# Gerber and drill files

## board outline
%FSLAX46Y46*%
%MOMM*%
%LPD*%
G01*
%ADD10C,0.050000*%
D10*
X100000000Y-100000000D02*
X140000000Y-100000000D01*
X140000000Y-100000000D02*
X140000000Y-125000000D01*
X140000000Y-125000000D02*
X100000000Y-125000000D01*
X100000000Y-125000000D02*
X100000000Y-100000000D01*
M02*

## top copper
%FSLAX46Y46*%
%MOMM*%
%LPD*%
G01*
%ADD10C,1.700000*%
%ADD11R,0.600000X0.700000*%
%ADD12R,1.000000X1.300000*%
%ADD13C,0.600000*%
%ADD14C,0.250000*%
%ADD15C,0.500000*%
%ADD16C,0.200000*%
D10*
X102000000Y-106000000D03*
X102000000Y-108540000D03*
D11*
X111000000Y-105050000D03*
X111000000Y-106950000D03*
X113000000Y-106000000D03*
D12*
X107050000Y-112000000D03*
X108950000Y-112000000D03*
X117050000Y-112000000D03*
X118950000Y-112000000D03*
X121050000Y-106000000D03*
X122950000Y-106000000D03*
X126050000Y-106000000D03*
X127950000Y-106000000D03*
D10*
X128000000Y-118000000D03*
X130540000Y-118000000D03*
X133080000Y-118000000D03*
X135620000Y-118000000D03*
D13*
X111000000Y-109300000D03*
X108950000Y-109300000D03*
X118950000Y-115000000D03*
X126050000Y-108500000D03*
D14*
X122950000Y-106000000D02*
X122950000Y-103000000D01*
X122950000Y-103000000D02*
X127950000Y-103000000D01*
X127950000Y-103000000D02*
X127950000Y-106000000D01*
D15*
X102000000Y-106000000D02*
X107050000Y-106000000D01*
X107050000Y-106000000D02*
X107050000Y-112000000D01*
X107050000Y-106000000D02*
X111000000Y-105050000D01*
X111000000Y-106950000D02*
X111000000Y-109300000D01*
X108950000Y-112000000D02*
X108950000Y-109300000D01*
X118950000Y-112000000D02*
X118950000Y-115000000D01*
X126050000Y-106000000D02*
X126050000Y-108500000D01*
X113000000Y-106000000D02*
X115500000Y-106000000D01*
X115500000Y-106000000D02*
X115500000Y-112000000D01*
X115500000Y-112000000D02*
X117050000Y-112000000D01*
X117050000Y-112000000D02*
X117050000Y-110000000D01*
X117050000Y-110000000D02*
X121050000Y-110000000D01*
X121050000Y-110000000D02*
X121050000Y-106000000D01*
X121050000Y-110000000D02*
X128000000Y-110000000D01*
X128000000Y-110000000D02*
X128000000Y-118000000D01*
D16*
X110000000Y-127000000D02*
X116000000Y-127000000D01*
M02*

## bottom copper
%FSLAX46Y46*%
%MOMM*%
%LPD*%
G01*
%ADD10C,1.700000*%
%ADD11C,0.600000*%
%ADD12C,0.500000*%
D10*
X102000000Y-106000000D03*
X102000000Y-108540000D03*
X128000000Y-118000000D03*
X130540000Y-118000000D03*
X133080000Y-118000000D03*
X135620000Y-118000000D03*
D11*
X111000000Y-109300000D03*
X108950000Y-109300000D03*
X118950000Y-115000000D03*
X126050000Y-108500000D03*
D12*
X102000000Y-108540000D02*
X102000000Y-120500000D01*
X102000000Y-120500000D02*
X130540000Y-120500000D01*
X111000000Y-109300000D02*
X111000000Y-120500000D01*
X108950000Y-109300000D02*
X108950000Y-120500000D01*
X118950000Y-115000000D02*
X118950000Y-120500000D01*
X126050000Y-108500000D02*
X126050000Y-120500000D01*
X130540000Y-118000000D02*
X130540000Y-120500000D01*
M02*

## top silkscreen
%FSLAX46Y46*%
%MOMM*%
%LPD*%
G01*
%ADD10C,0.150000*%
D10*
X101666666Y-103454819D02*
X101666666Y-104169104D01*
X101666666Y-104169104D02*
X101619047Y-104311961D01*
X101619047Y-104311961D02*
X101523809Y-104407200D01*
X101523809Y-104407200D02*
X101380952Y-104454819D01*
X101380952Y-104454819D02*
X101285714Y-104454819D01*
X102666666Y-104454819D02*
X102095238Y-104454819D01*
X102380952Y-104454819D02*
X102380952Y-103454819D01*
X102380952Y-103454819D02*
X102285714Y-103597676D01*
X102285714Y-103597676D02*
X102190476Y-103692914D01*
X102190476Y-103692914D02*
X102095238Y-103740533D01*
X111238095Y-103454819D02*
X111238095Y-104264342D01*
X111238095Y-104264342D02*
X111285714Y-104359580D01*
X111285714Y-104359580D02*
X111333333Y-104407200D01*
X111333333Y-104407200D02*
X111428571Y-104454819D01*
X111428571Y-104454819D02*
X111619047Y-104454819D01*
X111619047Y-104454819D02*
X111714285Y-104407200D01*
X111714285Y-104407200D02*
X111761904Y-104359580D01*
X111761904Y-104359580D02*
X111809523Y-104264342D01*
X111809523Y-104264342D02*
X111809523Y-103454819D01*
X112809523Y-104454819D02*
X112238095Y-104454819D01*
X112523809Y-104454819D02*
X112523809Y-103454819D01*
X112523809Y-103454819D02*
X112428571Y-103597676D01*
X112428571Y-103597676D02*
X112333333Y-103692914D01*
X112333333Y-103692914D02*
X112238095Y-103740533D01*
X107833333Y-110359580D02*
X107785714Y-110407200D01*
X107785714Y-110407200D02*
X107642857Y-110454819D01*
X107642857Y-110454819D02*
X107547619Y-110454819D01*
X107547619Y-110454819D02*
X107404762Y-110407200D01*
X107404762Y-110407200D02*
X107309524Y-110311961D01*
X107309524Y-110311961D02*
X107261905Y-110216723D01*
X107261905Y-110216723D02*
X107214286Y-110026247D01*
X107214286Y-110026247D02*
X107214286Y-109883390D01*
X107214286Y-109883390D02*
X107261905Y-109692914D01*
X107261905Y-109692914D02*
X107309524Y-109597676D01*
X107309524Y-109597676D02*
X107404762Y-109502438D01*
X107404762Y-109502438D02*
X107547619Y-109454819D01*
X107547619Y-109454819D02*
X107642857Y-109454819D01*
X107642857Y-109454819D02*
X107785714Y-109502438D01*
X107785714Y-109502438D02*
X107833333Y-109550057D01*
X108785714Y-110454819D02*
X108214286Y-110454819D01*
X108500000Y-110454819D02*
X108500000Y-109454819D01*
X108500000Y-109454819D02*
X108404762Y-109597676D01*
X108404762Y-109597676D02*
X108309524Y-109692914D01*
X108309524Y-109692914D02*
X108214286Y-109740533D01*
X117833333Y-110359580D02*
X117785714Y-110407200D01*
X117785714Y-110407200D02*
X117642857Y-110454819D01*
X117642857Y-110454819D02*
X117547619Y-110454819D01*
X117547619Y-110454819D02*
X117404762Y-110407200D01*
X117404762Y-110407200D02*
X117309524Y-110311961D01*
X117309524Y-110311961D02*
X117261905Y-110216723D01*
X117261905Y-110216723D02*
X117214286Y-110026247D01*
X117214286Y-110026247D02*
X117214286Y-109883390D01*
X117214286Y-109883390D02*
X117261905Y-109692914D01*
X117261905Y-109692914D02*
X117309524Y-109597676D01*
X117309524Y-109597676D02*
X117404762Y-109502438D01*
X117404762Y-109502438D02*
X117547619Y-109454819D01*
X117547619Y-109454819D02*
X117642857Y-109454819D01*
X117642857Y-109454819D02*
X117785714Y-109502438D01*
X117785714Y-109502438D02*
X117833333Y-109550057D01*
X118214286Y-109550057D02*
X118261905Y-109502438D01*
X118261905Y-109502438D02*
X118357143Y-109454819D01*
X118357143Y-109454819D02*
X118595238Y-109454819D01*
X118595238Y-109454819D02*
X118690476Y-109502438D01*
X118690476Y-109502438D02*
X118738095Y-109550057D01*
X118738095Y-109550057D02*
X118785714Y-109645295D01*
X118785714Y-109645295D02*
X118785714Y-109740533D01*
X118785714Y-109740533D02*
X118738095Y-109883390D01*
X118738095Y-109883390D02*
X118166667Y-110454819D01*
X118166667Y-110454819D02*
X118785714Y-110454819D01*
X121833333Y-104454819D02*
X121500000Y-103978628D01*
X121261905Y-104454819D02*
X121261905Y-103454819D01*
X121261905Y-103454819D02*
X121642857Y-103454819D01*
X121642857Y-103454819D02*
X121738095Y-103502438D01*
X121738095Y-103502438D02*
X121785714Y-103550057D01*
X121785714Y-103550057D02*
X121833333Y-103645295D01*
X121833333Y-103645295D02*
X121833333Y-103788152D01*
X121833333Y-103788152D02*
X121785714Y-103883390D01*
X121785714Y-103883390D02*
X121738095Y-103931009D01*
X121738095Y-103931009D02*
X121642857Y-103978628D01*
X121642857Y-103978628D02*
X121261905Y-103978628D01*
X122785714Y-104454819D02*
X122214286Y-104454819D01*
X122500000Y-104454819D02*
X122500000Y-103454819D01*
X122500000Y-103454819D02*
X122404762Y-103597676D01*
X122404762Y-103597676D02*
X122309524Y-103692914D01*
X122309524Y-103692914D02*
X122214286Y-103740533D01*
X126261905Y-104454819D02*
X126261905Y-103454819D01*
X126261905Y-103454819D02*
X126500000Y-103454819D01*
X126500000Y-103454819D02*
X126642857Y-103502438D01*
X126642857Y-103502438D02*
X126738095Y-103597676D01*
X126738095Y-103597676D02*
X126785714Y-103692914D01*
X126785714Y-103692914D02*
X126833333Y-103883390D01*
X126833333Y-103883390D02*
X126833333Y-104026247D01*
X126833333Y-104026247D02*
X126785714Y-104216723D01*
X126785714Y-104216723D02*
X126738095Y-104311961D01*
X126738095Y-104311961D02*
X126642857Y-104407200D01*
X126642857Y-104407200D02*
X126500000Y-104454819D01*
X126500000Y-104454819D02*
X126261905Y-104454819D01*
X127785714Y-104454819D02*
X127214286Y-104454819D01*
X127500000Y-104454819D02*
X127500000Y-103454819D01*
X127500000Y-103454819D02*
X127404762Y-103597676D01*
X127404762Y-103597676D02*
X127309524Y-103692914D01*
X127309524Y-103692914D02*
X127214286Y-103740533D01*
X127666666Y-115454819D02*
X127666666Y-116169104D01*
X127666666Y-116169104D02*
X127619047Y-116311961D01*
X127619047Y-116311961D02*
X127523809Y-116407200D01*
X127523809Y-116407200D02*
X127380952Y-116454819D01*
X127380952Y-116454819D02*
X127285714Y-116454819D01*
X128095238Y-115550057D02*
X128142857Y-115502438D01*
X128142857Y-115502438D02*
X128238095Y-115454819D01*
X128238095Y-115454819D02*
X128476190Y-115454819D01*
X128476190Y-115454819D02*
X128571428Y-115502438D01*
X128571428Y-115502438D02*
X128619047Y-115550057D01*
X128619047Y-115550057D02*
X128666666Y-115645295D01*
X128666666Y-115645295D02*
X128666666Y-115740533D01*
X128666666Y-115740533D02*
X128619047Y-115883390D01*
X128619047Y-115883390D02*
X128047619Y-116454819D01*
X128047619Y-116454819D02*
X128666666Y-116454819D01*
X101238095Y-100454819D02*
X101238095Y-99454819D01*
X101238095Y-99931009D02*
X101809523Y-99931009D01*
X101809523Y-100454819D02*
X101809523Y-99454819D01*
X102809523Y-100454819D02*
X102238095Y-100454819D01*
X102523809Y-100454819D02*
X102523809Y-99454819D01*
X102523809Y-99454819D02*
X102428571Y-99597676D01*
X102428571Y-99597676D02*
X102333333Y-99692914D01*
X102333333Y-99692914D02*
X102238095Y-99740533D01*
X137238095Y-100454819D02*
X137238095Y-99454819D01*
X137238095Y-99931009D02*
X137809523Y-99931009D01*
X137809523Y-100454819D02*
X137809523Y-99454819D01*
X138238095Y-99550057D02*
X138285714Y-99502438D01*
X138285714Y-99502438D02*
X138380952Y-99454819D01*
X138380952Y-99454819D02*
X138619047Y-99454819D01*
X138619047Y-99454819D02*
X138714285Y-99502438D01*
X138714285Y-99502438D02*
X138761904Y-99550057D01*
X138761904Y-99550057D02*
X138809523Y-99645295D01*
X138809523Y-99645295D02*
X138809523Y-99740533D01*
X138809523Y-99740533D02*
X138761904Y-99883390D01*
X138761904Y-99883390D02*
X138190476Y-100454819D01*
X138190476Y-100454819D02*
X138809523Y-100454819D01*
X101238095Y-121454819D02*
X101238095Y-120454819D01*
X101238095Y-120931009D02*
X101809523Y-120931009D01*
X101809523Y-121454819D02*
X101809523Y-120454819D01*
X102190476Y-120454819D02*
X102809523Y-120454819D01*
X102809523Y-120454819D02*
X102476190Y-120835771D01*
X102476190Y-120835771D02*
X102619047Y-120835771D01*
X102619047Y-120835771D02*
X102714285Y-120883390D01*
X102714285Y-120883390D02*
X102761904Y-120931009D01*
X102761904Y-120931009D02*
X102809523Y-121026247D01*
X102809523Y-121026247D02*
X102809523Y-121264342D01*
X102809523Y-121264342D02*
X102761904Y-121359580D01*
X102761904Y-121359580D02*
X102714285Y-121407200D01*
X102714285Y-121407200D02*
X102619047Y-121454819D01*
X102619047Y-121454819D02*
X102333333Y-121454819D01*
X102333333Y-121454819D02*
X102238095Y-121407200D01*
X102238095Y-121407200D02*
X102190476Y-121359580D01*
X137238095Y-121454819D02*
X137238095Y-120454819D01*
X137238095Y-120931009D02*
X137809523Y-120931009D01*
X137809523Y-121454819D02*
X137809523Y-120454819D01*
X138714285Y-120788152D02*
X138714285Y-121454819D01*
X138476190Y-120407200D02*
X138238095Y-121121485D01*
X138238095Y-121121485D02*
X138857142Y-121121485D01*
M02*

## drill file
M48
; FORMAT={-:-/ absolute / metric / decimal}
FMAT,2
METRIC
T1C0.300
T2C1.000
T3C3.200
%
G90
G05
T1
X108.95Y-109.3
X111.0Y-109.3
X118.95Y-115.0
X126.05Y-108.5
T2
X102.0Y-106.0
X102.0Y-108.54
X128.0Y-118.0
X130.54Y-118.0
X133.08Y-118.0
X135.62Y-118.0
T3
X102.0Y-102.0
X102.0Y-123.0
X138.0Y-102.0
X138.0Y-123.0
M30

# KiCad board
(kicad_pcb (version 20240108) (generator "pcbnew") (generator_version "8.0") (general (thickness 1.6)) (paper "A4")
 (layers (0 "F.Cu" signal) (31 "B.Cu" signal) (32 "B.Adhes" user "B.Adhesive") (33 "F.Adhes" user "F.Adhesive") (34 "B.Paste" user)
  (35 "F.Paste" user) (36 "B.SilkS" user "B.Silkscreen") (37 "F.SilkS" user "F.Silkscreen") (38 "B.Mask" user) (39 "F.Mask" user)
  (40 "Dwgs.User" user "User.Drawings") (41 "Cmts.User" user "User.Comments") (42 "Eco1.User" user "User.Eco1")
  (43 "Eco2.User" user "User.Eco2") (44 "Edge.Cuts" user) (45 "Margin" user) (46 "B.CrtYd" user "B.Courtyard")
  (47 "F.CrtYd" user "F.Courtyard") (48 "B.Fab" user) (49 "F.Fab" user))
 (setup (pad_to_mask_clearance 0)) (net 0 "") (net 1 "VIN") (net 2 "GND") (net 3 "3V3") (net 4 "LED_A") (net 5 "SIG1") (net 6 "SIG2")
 (gr_line (start 100 100) (end 140 100) (stroke (width 0.05) (type default)) (layer "Edge.Cuts"))
 (gr_line (start 140 100) (end 140 125) (stroke (width 0.05) (type default)) (layer "Edge.Cuts"))
 (gr_line (start 140 125) (end 100 125) (stroke (width 0.05) (type default)) (layer "Edge.Cuts"))
 (gr_line (start 100 125) (end 100 100) (stroke (width 0.05) (type default)) (layer "Edge.Cuts"))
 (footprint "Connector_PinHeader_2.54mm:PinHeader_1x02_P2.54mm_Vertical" (layer "F.Cu") (at 102 106)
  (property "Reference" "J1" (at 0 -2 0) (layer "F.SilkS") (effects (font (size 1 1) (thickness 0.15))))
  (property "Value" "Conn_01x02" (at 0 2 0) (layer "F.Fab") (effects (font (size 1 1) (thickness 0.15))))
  (pad "1" thru_hole circle (at 0 0) (size 1.7 1.7) (drill 1) (layers "*.Cu" "*.Mask") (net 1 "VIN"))
  (pad "2" thru_hole circle (at 0 2.54) (size 1.7 1.7) (drill 1) (layers "*.Cu" "*.Mask") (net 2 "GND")))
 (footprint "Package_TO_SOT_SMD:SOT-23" (layer "F.Cu") (at 112 106)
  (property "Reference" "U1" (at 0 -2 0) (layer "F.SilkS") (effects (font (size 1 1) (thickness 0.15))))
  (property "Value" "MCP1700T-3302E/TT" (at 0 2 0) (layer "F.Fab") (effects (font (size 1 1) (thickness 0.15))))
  (pad "1" smd rect (at -1 -0.95) (size 0.6 0.7) (layers "F.Cu" "F.Paste" "F.Mask") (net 1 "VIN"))
  (pad "2" smd rect (at -1 0.95) (size 0.6 0.7) (layers "F.Cu" "F.Paste" "F.Mask") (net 2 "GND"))
  (pad "3" smd rect (at 1 0) (size 0.6 0.7) (layers "F.Cu" "F.Paste" "F.Mask") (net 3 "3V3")))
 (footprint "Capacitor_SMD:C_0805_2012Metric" (layer "F.Cu") (at 108 112)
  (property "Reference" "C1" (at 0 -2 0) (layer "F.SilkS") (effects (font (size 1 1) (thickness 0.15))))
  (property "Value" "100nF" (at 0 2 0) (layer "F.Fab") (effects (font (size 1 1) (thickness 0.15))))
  (pad "1" smd rect (at -0.95 0) (size 1 1.3) (layers "F.Cu" "F.Paste" "F.Mask") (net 1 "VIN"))
  (pad "2" smd rect (at 0.95 0) (size 1 1.3) (layers "F.Cu" "F.Paste" "F.Mask") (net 2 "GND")))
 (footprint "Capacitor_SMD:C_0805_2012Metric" (layer "F.Cu") (at 118 112)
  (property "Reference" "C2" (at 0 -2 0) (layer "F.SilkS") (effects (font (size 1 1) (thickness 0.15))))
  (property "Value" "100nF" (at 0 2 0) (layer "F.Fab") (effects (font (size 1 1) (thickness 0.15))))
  (pad "1" smd rect (at -0.95 0) (size 1 1.3) (layers "F.Cu" "F.Paste" "F.Mask") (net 3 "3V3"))
  (pad "2" smd rect (at 0.95 0) (size 1 1.3) (layers "F.Cu" "F.Paste" "F.Mask") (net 2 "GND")))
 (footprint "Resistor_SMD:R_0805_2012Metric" (layer "F.Cu") (at 122 106)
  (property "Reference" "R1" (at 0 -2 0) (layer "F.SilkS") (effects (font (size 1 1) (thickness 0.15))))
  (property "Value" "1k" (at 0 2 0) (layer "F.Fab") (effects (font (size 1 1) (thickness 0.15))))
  (pad "1" smd rect (at -0.95 0) (size 1 1.3) (layers "F.Cu" "F.Paste" "F.Mask") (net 3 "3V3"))
  (pad "2" smd rect (at 0.95 0) (size 1 1.3) (layers "F.Cu" "F.Paste" "F.Mask") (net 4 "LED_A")))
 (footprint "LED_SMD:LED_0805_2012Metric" (layer "F.Cu") (at 127 106)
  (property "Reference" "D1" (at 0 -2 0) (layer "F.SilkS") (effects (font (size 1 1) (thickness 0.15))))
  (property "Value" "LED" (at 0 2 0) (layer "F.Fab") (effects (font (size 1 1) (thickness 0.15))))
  (pad "1" smd rect (at -0.95 0) (size 1 1.3) (layers "F.Cu" "F.Paste" "F.Mask") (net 2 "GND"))
  (pad "2" smd rect (at 0.95 0) (size 1 1.3) (layers "F.Cu" "F.Paste" "F.Mask") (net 4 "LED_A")))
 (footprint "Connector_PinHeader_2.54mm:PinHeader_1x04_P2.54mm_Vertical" (layer "F.Cu") (at 128 118)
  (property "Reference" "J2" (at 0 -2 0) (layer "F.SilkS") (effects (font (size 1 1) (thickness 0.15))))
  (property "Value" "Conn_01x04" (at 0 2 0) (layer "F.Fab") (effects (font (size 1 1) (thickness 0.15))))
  (pad "1" thru_hole circle (at 0 0) (size 1.7 1.7) (drill 1) (layers "*.Cu" "*.Mask") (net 3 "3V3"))
  (pad "2" thru_hole circle (at 2.54 0) (size 1.7 1.7) (drill 1) (layers "*.Cu" "*.Mask") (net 2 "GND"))
  (pad "3" thru_hole circle (at 5.08 0) (size 1.7 1.7) (drill 1) (layers "*.Cu" "*.Mask") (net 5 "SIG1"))
  (pad "4" thru_hole circle (at 7.62 0) (size 1.7 1.7) (drill 1) (layers "*.Cu" "*.Mask") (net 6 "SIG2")))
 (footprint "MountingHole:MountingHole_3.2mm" (layer "F.Cu") (at 102 102)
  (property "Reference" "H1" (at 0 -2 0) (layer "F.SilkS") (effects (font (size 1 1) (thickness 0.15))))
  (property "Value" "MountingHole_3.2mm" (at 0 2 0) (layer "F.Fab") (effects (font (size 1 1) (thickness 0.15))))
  (pad "1" np_thru_hole circle (at 0 0) (size 3.2 3.2) (drill 3.2) (layers "*.Cu" "*.Mask")))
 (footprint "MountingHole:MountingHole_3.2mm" (layer "F.Cu") (at 138 102)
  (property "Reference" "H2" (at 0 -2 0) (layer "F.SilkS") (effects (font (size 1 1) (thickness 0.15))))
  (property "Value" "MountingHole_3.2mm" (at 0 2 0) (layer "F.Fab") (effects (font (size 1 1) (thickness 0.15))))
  (pad "1" np_thru_hole circle (at 0 0) (size 3.2 3.2) (drill 3.2) (layers "*.Cu" "*.Mask")))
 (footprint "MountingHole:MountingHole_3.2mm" (layer "F.Cu") (at 102 123)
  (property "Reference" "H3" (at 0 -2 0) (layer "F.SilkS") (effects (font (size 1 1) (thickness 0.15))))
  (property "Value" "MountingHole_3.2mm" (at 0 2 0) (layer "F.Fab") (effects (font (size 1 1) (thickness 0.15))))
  (pad "1" np_thru_hole circle (at 0 0) (size 3.2 3.2) (drill 3.2) (layers "*.Cu" "*.Mask")))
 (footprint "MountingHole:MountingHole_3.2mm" (layer "F.Cu") (at 138 123)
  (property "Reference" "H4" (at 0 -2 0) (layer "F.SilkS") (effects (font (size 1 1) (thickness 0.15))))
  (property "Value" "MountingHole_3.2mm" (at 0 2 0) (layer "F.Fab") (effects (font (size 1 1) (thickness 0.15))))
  (pad "1" np_thru_hole circle (at 0 0) (size 3.2 3.2) (drill 3.2) (layers "*.Cu" "*.Mask")))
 (segment (start 122.95 106) (end 122.95 103) (width 0.25) (layer "F.Cu") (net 4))
 (segment (start 122.95 103) (end 127.95 103) (width 0.25) (layer "F.Cu") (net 4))
 (segment (start 127.95 103) (end 127.95 106) (width 0.25) (layer "F.Cu") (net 4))
 (segment (start 102 106) (end 107.05 106) (width 0.5) (layer "F.Cu") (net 1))
 (segment (start 107.05 106) (end 107.05 112) (width 0.5) (layer "F.Cu") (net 1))
 (segment (start 107.05 106) (end 111 105.05) (width 0.5) (layer "F.Cu") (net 1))
 (segment (start 111 106.95) (end 111 109.3) (width 0.5) (layer "F.Cu") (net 2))
 (segment (start 108.95 112) (end 108.95 109.3) (width 0.5) (layer "F.Cu") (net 2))
 (segment (start 118.95 112) (end 118.95 115) (width 0.5) (layer "F.Cu") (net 2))
 (segment (start 126.05 106) (end 126.05 108.5) (width 0.5) (layer "F.Cu") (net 2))
 (segment (start 113 106) (end 115.5 106) (width 0.5) (layer "F.Cu") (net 3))
 (segment (start 115.5 106) (end 115.5 112) (width 0.5) (layer "F.Cu") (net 3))
 (segment (start 115.5 112) (end 117.05 112) (width 0.5) (layer "F.Cu") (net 3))
 (segment (start 117.05 112) (end 117.05 110) (width 0.5) (layer "F.Cu") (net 3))
 (segment (start 117.05 110) (end 121.05 110) (width 0.5) (layer "F.Cu") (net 3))
 (segment (start 121.05 110) (end 121.05 106) (width 0.5) (layer "F.Cu") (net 3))
 (segment (start 121.05 110) (end 128 110) (width 0.5) (layer "F.Cu") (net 3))
 (segment (start 128 110) (end 128 118) (width 0.5) (layer "F.Cu") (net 3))
 (segment (start 102 108.54) (end 102 120.5) (width 0.5) (layer "B.Cu") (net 2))
 (segment (start 102 120.5) (end 130.54 120.5) (width 0.5) (layer "B.Cu") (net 2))
 (segment (start 111 109.3) (end 111 120.5) (width 0.5) (layer "B.Cu") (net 2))
 (segment (start 108.95 109.3) (end 108.95 120.5) (width 0.5) (layer "B.Cu") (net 2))
 (segment (start 118.95 115) (end 118.95 120.5) (width 0.5) (layer "B.Cu") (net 2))
 (segment (start 126.05 108.5) (end 126.05 120.5) (width 0.5) (layer "B.Cu") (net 2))
 (segment (start 130.54 118) (end 130.54 120.5) (width 0.5) (layer "B.Cu") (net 2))
 (via (at 111 109.3) (size 0.6) (drill 0.3) (layers "F.Cu" "B.Cu") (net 2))
 (via (at 108.95 109.3) (size 0.6) (drill 0.3) (layers "F.Cu" "B.Cu") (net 2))
 (via (at 118.95 115) (size 0.6) (drill 0.3) (layers "F.Cu" "B.Cu") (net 2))
 (via (at 126.05 108.5) (size 0.6) (drill 0.3) (layers "F.Cu" "B.Cu") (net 2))
 (segment (start 110 127) (end 116 127) (width 0.2) (layer "F.Cu") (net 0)))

